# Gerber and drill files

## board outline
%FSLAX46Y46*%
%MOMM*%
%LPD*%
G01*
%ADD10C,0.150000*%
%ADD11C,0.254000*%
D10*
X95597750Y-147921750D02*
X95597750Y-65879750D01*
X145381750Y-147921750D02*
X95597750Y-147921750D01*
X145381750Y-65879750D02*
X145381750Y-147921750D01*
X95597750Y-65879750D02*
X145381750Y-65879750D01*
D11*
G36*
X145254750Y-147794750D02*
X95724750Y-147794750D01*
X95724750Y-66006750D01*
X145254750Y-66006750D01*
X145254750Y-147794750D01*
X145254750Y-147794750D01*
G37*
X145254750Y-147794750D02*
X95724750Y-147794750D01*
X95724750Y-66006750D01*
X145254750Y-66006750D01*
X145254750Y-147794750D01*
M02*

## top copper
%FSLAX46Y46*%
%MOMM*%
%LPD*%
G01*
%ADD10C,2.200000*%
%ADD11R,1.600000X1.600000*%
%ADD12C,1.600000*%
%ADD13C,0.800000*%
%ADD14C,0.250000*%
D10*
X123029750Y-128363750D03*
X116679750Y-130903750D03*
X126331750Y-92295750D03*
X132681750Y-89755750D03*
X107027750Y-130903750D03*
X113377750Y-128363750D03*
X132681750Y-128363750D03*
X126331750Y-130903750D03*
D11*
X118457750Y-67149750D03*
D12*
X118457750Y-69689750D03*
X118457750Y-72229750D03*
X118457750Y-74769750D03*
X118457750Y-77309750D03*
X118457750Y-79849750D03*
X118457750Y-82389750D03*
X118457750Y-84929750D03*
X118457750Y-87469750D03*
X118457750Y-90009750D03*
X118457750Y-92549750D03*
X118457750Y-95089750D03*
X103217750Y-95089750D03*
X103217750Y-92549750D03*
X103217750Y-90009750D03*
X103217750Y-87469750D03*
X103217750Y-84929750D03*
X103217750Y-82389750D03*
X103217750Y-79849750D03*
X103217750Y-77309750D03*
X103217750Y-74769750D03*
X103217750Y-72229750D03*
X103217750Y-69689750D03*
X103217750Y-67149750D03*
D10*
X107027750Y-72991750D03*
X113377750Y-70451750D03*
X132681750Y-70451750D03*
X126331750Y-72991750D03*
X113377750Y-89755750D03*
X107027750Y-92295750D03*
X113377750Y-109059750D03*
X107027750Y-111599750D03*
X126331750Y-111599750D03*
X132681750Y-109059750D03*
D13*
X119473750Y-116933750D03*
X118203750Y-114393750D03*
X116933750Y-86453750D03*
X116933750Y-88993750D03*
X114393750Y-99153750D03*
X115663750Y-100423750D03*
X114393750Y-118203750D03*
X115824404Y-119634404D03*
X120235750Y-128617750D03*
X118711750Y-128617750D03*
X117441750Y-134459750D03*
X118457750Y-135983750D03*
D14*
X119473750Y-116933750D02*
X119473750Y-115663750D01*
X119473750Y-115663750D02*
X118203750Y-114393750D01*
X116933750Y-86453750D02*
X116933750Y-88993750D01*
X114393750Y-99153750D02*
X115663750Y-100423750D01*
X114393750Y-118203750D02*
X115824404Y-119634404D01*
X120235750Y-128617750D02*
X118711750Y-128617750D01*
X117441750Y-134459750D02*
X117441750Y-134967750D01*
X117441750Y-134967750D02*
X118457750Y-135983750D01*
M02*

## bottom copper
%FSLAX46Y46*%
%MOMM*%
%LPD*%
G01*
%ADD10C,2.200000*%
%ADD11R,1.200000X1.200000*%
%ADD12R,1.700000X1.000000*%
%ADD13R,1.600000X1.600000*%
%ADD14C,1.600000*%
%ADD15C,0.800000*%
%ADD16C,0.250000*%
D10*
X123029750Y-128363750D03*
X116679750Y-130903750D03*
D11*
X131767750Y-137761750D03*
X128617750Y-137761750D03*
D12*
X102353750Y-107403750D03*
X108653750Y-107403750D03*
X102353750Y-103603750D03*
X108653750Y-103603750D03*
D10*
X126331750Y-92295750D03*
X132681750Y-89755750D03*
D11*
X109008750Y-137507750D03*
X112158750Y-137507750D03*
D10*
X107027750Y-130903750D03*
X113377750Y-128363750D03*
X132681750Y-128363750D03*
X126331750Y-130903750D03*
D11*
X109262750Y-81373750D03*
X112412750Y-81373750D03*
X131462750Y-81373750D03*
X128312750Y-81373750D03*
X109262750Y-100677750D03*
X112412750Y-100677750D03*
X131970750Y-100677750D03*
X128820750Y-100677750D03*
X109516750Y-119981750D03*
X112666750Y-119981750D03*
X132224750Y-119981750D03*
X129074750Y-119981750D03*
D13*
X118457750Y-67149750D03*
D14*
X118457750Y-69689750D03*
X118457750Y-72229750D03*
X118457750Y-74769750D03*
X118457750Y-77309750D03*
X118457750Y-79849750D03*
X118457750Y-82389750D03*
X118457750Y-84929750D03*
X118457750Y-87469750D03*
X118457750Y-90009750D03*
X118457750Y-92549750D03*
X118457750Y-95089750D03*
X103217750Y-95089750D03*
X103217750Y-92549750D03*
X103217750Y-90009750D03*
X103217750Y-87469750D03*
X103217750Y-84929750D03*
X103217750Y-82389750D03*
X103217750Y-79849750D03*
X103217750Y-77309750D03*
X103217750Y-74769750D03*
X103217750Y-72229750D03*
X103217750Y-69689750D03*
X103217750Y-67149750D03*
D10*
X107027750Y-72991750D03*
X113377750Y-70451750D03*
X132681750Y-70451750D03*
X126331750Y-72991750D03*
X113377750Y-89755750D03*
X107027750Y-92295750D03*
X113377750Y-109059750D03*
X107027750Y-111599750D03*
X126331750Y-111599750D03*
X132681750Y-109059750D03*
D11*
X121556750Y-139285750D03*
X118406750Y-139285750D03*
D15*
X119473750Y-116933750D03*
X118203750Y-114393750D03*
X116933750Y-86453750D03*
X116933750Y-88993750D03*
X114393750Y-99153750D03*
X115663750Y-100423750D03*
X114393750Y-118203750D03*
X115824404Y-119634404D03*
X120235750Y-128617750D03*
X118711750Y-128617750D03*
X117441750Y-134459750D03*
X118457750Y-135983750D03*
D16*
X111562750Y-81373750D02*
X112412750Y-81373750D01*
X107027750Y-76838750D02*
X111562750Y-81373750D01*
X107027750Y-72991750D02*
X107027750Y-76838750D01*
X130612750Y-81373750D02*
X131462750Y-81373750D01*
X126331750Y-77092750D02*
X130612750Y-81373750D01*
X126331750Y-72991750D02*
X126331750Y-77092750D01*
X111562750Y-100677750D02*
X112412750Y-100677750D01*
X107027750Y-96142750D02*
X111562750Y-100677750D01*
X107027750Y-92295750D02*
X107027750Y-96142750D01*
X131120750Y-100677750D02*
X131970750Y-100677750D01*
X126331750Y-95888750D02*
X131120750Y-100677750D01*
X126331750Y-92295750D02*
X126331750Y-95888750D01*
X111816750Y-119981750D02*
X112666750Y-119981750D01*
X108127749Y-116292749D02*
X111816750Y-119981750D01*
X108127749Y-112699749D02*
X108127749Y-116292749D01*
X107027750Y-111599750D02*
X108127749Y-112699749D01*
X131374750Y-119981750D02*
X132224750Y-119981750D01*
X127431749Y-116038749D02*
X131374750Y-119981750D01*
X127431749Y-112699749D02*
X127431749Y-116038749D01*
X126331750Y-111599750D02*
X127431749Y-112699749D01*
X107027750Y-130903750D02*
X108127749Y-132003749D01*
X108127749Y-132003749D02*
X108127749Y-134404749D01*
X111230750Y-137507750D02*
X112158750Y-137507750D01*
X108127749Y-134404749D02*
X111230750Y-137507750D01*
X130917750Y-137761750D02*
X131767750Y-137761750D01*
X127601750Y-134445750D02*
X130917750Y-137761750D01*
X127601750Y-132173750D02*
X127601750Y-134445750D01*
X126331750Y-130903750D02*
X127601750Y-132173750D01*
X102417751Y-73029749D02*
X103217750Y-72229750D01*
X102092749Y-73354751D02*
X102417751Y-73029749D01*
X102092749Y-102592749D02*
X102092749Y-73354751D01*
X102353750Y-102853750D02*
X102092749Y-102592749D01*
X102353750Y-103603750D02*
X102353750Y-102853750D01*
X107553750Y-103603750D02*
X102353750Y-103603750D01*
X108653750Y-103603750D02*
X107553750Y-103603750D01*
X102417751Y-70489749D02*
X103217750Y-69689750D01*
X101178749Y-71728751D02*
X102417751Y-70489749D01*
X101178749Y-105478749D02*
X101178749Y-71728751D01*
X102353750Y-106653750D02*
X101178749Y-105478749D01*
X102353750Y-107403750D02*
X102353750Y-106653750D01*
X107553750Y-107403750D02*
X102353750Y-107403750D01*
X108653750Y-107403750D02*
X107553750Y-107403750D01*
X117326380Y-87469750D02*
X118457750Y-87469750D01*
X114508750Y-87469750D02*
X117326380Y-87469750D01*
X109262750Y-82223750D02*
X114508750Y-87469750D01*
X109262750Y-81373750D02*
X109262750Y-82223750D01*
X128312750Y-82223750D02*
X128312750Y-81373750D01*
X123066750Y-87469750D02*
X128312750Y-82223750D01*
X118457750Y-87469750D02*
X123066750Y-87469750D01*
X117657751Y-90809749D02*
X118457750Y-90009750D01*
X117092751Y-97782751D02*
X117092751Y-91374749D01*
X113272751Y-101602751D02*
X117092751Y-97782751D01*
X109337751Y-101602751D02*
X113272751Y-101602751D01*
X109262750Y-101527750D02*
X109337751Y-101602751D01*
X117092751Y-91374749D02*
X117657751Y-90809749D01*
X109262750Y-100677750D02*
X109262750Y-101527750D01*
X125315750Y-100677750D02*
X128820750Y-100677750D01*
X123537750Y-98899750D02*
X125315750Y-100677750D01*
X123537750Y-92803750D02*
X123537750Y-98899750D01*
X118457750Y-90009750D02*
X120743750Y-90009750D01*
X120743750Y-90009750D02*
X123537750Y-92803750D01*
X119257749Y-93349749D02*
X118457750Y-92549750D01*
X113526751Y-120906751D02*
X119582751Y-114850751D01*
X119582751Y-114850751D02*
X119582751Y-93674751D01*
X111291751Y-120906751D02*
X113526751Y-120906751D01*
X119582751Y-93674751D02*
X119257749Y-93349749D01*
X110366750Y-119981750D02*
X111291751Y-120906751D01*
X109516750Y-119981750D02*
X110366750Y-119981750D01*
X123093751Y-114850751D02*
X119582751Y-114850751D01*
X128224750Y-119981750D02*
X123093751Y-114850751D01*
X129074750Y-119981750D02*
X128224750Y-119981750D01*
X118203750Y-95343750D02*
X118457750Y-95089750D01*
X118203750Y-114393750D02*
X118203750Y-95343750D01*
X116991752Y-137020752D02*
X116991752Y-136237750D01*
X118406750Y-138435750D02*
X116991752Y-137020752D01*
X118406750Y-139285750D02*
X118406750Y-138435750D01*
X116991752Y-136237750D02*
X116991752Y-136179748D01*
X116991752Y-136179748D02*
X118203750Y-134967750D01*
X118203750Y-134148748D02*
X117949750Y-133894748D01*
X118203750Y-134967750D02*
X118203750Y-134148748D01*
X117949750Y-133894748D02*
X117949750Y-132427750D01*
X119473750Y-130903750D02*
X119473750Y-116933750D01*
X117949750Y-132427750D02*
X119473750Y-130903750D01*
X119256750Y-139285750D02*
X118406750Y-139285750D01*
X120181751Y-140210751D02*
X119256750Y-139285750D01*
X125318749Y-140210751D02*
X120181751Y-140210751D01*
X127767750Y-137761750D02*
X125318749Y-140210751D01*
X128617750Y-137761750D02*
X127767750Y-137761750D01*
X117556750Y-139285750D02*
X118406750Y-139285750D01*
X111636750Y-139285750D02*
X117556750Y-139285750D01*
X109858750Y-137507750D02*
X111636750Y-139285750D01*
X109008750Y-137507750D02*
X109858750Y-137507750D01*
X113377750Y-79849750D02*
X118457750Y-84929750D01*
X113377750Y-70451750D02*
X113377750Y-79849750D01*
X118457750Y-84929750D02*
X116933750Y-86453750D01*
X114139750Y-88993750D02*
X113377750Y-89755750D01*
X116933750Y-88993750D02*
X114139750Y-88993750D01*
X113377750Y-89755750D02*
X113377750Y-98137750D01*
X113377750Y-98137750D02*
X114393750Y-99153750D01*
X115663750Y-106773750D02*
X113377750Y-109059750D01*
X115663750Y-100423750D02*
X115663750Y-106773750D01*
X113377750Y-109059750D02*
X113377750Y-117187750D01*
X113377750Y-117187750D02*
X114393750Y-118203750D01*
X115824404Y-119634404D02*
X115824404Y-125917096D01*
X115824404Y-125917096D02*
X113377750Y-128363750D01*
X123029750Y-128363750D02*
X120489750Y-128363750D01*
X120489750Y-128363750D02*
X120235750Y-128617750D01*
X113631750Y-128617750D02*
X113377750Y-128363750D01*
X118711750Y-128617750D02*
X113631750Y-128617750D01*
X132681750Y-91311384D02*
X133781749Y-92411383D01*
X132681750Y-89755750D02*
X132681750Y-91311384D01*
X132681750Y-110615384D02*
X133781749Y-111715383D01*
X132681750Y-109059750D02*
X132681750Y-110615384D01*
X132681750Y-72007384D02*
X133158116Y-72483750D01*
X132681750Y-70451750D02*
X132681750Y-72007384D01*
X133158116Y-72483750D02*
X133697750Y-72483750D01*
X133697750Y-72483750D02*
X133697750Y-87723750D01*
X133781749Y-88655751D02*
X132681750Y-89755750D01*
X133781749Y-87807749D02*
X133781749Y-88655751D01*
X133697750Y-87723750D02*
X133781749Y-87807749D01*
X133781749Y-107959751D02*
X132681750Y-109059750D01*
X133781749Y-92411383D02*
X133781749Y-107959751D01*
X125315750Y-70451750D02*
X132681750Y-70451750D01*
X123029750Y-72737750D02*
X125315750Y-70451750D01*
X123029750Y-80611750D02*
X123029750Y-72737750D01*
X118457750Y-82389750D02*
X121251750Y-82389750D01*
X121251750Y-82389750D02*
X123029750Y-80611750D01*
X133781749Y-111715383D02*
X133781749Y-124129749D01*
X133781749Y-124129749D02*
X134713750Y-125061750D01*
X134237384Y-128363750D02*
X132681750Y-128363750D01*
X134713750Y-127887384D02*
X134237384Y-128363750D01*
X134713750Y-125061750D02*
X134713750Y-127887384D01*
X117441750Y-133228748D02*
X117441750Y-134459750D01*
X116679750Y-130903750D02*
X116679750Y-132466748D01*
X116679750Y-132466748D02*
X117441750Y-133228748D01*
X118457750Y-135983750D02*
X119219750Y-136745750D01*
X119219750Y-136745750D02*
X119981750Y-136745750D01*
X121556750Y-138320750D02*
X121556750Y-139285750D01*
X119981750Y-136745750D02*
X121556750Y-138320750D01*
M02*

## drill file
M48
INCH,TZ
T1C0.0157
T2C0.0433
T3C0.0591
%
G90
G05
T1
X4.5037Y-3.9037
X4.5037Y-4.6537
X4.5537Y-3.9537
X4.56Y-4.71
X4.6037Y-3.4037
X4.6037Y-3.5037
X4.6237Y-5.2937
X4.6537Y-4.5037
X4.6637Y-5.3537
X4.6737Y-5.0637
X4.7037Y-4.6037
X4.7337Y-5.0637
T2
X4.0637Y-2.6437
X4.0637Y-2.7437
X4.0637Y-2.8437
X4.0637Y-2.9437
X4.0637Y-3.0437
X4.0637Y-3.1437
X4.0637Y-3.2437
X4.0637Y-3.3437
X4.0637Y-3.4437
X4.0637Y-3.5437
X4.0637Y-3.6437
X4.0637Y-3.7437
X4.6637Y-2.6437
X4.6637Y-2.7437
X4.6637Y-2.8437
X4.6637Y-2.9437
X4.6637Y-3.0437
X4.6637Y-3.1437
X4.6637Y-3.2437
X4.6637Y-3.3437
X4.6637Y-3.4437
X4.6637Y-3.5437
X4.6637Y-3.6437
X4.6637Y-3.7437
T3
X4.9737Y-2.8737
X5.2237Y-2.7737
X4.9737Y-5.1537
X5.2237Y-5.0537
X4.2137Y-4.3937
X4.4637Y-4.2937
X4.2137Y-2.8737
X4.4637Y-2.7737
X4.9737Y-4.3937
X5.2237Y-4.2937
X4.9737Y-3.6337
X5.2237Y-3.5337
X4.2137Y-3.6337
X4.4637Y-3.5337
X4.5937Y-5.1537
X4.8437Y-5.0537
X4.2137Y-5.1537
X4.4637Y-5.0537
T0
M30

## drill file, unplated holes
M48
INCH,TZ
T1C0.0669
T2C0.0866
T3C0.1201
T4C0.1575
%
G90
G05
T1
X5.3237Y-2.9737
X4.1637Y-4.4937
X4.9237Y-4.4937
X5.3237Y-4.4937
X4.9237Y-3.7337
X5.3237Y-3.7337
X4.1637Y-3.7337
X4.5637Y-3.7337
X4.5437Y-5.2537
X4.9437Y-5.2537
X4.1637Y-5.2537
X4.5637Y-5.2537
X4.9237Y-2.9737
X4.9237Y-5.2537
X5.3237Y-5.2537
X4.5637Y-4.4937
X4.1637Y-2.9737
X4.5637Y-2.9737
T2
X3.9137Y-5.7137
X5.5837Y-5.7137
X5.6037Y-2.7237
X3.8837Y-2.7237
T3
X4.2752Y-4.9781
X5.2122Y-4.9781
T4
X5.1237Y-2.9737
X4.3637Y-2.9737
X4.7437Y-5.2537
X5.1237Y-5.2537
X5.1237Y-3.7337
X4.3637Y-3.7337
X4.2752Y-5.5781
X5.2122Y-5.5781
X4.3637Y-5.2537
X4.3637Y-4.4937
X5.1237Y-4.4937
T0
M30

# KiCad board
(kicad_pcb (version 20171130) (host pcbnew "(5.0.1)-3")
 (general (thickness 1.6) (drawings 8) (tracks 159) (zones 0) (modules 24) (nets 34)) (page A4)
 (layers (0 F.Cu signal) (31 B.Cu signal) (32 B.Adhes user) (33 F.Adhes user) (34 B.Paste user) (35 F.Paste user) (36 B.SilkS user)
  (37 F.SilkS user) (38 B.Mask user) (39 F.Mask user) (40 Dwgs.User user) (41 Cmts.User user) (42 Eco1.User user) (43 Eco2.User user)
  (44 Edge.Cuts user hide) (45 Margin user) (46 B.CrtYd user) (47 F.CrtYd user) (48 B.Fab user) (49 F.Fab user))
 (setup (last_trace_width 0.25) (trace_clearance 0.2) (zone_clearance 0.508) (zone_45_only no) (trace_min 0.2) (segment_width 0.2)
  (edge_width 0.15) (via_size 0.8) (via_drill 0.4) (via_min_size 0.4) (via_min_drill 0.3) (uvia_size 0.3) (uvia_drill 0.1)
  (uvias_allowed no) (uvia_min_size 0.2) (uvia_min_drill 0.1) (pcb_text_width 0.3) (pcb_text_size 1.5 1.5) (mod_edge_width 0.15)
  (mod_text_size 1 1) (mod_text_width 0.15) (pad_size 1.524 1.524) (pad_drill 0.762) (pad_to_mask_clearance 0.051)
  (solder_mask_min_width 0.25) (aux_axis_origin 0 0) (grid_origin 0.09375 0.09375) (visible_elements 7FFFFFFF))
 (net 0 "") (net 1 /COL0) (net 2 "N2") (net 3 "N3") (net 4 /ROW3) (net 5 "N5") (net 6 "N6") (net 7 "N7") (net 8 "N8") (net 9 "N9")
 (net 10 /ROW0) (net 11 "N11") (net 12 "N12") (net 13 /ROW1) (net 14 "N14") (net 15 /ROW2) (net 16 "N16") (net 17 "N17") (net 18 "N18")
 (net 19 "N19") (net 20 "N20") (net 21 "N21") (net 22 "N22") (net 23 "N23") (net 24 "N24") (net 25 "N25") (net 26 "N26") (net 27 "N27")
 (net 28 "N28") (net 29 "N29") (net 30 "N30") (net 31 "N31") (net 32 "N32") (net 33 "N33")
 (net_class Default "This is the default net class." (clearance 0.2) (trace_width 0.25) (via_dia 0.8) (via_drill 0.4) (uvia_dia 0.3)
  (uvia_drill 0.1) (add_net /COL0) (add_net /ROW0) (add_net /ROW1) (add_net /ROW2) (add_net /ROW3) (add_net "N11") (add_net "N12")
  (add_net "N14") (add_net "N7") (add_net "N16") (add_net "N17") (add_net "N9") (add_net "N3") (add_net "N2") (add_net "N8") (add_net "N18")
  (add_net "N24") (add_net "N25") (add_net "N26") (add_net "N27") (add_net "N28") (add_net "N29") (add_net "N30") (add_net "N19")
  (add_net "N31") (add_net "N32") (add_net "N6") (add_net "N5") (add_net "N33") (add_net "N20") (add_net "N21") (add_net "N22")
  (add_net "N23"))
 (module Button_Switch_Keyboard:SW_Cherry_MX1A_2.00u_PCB (layer F.Cu) (at 123.02975 128.36375)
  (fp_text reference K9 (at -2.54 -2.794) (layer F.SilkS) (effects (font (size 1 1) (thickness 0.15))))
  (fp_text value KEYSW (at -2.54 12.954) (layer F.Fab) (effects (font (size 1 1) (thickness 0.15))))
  (pad 1 thru_hole circle (at 0 0) (size 2.2 2.2) (drill 1.5) (layers *.Cu *.Mask) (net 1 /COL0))
  (pad 2 thru_hole circle (at -6.35 2.54) (size 2.2 2.2) (drill 1.5) (layers *.Cu *.Mask) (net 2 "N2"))
  (pad "" np_thru_hole circle (at -2.54 5.08) (size 4 4) (drill 4) (layers *.Cu *.Mask))
  (pad "" np_thru_hole circle (at -7.62 5.08) (size 1.7 1.7) (drill 1.7) (layers *.Cu *.Mask))
  (pad "" np_thru_hole circle (at 2.54 5.08) (size 1.7 1.7) (drill 1.7) (layers *.Cu *.Mask))
  (pad "" np_thru_hole circle (at 9.36 13.32) (size 4 4) (drill 4) (layers *.Cu *.Mask))
  (pad "" np_thru_hole circle (at -14.44 13.32) (size 4 4) (drill 4) (layers *.Cu *.Mask))
  (pad "" np_thru_hole circle (at -14.44 -1.92) (size 3.05 3.05) (drill 3.05) (layers *.Cu *.Mask))
  (pad "" np_thru_hole circle (at 9.36 -1.92) (size 3.05 3.05) (drill 3.05) (layers *.Cu *.Mask)))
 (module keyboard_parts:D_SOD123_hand (layer B.Cu) (at 130.19275 137.76175)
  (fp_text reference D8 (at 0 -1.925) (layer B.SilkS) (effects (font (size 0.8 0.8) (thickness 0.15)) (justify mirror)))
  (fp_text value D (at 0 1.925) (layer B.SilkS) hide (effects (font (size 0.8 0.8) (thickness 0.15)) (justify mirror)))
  (pad 2 smd rect (at 1.575 0) (size 1.2 1.2) (layers B.Cu B.Paste B.Mask) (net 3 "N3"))
  (pad 1 smd rect (at -1.575 0) (size 1.2 1.2) (layers B.Cu B.Paste B.Mask) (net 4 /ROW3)))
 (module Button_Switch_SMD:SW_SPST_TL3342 (layer B.Cu) (at 105.50375 105.50375)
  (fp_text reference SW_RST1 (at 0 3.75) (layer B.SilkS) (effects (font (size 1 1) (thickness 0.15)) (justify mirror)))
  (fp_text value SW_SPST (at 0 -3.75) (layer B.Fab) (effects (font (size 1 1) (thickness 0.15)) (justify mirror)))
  (pad 1 smd rect (at -3.15 1.9) (size 1.7 1) (layers B.Cu B.Paste B.Mask) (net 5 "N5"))
  (pad 1 smd rect (at 3.15 1.9) (size 1.7 1) (layers B.Cu B.Paste B.Mask) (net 5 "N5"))
  (pad 2 smd rect (at -3.15 -1.9) (size 1.7 1) (layers B.Cu B.Paste B.Mask) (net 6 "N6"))
  (pad 2 smd rect (at 3.15 -1.9) (size 1.7 1) (layers B.Cu B.Paste B.Mask) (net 6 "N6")))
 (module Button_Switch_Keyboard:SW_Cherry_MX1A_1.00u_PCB (layer F.Cu) (at 132.68175 89.75575)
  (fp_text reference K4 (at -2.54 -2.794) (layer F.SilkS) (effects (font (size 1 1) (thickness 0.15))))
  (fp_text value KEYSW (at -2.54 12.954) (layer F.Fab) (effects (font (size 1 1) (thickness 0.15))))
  (pad "" np_thru_hole circle (at 2.54 5.08) (size 1.7 1.7) (drill 1.7) (layers *.Cu *.Mask))
  (pad "" np_thru_hole circle (at -7.62 5.08) (size 1.7 1.7) (drill 1.7) (layers *.Cu *.Mask))
  (pad "" np_thru_hole circle (at -2.54 5.08) (size 4 4) (drill 4) (layers *.Cu *.Mask))
  (pad 2 thru_hole circle (at -6.35 2.54) (size 2.2 2.2) (drill 1.5) (layers *.Cu *.Mask) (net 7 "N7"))
  (pad 1 thru_hole circle (at 0 0) (size 2.2 2.2) (drill 1.5) (layers *.Cu *.Mask) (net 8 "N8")))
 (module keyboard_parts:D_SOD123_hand (layer B.Cu) (at 110.58375 137.50775)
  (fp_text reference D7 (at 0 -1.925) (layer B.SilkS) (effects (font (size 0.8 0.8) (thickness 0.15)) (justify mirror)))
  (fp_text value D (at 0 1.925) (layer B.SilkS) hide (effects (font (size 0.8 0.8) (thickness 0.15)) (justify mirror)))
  (pad 1 smd rect (at -1.575 0) (size 1.2 1.2) (layers B.Cu B.Paste B.Mask) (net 4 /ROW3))
  (pad 2 smd rect (at 1.575 0) (size 1.2 1.2) (layers B.Cu B.Paste B.Mask) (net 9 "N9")))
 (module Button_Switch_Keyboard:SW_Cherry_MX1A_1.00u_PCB (layer F.Cu) (at 113.37775 128.36375)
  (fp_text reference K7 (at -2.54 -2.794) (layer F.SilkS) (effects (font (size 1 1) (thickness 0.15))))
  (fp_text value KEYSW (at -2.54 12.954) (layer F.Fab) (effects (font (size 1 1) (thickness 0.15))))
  (pad "" np_thru_hole circle (at 2.54 5.08) (size 1.7 1.7) (drill 1.7) (layers *.Cu *.Mask))
  (pad "" np_thru_hole circle (at -7.62 5.08) (size 1.7 1.7) (drill 1.7) (layers *.Cu *.Mask))
  (pad "" np_thru_hole circle (at -2.54 5.08) (size 4 4) (drill 4) (layers *.Cu *.Mask))
  (pad 2 thru_hole circle (at -6.35 2.54) (size 2.2 2.2) (drill 1.5) (layers *.Cu *.Mask) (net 9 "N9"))
  (pad 1 thru_hole circle (at 0 0) (size 2.2 2.2) (drill 1.5) (layers *.Cu *.Mask) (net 1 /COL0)))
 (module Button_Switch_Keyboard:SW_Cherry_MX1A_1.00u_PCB (layer F.Cu) (at 132.68175 128.36375)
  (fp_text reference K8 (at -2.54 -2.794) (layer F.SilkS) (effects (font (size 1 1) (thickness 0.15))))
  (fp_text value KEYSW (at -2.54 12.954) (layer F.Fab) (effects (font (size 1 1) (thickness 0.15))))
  (pad 1 thru_hole circle (at 0 0) (size 2.2 2.2) (drill 1.5) (layers *.Cu *.Mask) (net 8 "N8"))
  (pad 2 thru_hole circle (at -6.35 2.54) (size 2.2 2.2) (drill 1.5) (layers *.Cu *.Mask) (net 3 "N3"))
  (pad "" np_thru_hole circle (at -2.54 5.08) (size 4 4) (drill 4) (layers *.Cu *.Mask))
  (pad "" np_thru_hole circle (at -7.62 5.08) (size 1.7 1.7) (drill 1.7) (layers *.Cu *.Mask))
  (pad "" np_thru_hole circle (at 2.54 5.08) (size 1.7 1.7) (drill 1.7) (layers *.Cu *.Mask)))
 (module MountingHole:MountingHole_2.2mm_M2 (layer F.Cu) (at 99.40775 145.12775)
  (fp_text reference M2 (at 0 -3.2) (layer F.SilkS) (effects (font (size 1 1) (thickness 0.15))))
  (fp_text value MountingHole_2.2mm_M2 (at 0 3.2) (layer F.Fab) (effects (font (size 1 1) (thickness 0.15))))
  (pad 1 np_thru_hole circle (at 0 0) (size 2.2 2.2) (drill 2.2) (layers *.Cu *.Mask)))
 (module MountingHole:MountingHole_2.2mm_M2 (layer F.Cu) (at 141.82575 145.12775)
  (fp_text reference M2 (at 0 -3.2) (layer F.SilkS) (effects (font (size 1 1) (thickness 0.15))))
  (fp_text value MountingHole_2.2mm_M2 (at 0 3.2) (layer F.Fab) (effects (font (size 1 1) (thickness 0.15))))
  (pad 1 np_thru_hole circle (at 0 0) (size 2.2 2.2) (drill 2.2) (layers *.Cu *.Mask)))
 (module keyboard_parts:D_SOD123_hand (layer B.Cu) (at 110.83775 81.37375)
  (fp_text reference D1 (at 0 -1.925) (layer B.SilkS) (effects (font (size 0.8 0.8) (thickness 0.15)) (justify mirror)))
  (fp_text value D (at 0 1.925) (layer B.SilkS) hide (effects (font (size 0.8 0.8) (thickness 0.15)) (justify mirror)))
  (pad 1 smd rect (at -1.575 0) (size 1.2 1.2) (layers B.Cu B.Paste B.Mask) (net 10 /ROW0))
  (pad 2 smd rect (at 1.575 0) (size 1.2 1.2) (layers B.Cu B.Paste B.Mask) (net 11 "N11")))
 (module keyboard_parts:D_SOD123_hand (layer B.Cu) (at 129.88775 81.37375)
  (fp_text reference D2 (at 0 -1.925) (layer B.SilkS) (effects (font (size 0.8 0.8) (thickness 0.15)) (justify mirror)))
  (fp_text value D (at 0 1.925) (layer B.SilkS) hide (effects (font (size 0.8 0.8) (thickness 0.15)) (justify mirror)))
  (pad 2 smd rect (at 1.575 0) (size 1.2 1.2) (layers B.Cu B.Paste B.Mask) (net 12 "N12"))
  (pad 1 smd rect (at -1.575 0) (size 1.2 1.2) (layers B.Cu B.Paste B.Mask) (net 10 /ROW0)))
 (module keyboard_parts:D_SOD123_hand (layer B.Cu) (at 110.83775 100.67775)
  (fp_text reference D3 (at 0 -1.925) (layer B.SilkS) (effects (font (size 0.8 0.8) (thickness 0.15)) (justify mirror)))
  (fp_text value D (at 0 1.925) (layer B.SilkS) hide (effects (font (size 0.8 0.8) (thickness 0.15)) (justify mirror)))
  (pad 1 smd rect (at -1.575 0) (size 1.2 1.2) (layers B.Cu B.Paste B.Mask) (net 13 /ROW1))
  (pad 2 smd rect (at 1.575 0) (size 1.2 1.2) (layers B.Cu B.Paste B.Mask) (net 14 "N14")))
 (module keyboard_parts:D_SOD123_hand (layer B.Cu) (at 130.39575 100.67775)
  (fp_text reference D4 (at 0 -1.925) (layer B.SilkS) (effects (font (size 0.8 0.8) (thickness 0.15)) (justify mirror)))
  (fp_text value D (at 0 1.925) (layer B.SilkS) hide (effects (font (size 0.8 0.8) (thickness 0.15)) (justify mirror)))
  (pad 2 smd rect (at 1.575 0) (size 1.2 1.2) (layers B.Cu B.Paste B.Mask) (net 7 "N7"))
  (pad 1 smd rect (at -1.575 0) (size 1.2 1.2) (layers B.Cu B.Paste B.Mask) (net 13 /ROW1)))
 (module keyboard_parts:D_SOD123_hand (layer B.Cu) (at 111.09175 119.98175)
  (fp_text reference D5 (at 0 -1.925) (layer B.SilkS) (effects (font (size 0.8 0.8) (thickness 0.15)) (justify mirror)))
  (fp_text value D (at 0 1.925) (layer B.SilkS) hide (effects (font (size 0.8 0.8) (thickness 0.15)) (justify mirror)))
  (pad 1 smd rect (at -1.575 0) (size 1.2 1.2) (layers B.Cu B.Paste B.Mask) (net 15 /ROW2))
  (pad 2 smd rect (at 1.575 0) (size 1.2 1.2) (layers B.Cu B.Paste B.Mask) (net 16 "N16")))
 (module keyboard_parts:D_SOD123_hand (layer B.Cu) (at 130.64975 119.98175)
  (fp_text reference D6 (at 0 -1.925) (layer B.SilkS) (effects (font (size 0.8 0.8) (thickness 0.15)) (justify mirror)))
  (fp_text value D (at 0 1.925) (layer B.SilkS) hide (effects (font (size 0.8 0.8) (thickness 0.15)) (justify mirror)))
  (pad 2 smd rect (at 1.575 0) (size 1.2 1.2) (layers B.Cu B.Paste B.Mask) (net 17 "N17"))
  (pad 1 smd rect (at -1.575 0) (size 1.2 1.2) (layers B.Cu B.Paste B.Mask) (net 15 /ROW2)))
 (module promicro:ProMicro (layer B.Cu) (at 110.83775 81.11975 270)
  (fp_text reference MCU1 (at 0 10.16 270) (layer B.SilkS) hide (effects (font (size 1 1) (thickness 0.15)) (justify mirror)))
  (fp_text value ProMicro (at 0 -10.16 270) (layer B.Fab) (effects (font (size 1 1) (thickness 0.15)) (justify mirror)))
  (pad 1 thru_hole rect (at -13.97 -7.62 270) (size 1.6 1.6) (drill 1.1) (layers *.Cu *.Mask B.SilkS) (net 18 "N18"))
  (pad 2 thru_hole circle (at -11.43 -7.62 270) (size 1.6 1.6) (drill 1.1) (layers *.Cu *.Mask B.SilkS) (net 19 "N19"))
  (pad 3 thru_hole circle (at -8.89 -7.62 270) (size 1.6 1.6) (drill 1.1) (layers *.Cu *.Mask B.SilkS) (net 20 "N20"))
  (pad 4 thru_hole circle (at -6.35 -7.62 270) (size 1.6 1.6) (drill 1.1) (layers *.Cu *.Mask B.SilkS) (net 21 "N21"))
  (pad 5 thru_hole circle (at -3.81 -7.62 270) (size 1.6 1.6) (drill 1.1) (layers *.Cu *.Mask B.SilkS) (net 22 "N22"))
  (pad 6 thru_hole circle (at -1.27 -7.62 270) (size 1.6 1.6) (drill 1.1) (layers *.Cu *.Mask B.SilkS) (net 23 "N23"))
  (pad 7 thru_hole circle (at 1.27 -7.62 270) (size 1.6 1.6) (drill 1.1) (layers *.Cu *.Mask B.SilkS) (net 8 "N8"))
  (pad 8 thru_hole circle (at 3.81 -7.62 270) (size 1.6 1.6) (drill 1.1) (layers *.Cu *.Mask B.SilkS) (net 1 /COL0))
  (pad 9 thru_hole circle (at 6.35 -7.62 270) (size 1.6 1.6) (drill 1.1) (layers *.Cu *.Mask B.SilkS) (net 10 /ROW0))
  (pad 10 thru_hole circle (at 8.89 -7.62 270) (size 1.6 1.6) (drill 1.1) (layers *.Cu *.Mask B.SilkS) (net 13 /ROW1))
  (pad 11 thru_hole circle (at 11.43 -7.62 270) (size 1.6 1.6) (drill 1.1) (layers *.Cu *.Mask B.SilkS) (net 15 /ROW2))
  (pad 12 thru_hole circle (at 13.97 -7.62 270) (size 1.6 1.6) (drill 1.1) (layers *.Cu *.Mask B.SilkS) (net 4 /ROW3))
  (pad 13 thru_hole circle (at 13.97 7.62 270) (size 1.6 1.6) (drill 1.1) (layers *.Cu *.Mask B.SilkS) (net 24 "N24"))
  (pad 14 thru_hole circle (at 11.43 7.62 270) (size 1.6 1.6) (drill 1.1) (layers *.Cu *.Mask B.SilkS) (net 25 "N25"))
  (pad 15 thru_hole circle (at 8.89 7.62 270) (size 1.6 1.6) (drill 1.1) (layers *.Cu *.Mask B.SilkS) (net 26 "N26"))
  (pad 16 thru_hole circle (at 6.35 7.62 270) (size 1.6 1.6) (drill 1.1) (layers *.Cu *.Mask B.SilkS) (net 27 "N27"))
  (pad 17 thru_hole circle (at 3.81 7.62 270) (size 1.6 1.6) (drill 1.1) (layers *.Cu *.Mask B.SilkS) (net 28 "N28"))
  (pad 18 thru_hole circle (at 1.27 7.62 270) (size 1.6 1.6) (drill 1.1) (layers *.Cu *.Mask B.SilkS) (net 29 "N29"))
  (pad 19 thru_hole circle (at -1.27 7.62 270) (size 1.6 1.6) (drill 1.1) (layers *.Cu *.Mask B.SilkS) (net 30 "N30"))
  (pad 20 thru_hole circle (at -3.81 7.62 270) (size 1.6 1.6) (drill 1.1) (layers *.Cu *.Mask B.SilkS) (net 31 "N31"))
  (pad 21 thru_hole circle (at -6.35 7.62 270) (size 1.6 1.6) (drill 1.1) (layers *.Cu *.Mask B.SilkS) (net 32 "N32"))
  (pad 22 thru_hole circle (at -8.89 7.62 270) (size 1.6 1.6) (drill 1.1) (layers *.Cu *.Mask B.SilkS) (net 6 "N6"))
  (pad 23 thru_hole circle (at -11.43 7.62 270) (size 1.6 1.6) (drill 1.1) (layers *.Cu *.Mask B.SilkS) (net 5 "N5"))
  (pad 24 thru_hole circle (at -13.97 7.62 270) (size 1.6 1.6) (drill 1.1) (layers *.Cu *.Mask B.SilkS) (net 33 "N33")))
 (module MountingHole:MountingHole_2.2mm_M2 (layer F.Cu) (at 142.33375 69.18175)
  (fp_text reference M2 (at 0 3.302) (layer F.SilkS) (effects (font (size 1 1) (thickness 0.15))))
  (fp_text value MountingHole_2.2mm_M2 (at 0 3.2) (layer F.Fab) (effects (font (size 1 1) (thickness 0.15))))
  (pad 1 np_thru_hole circle (at 0 0) (size 2.2 2.2) (drill 2.2) (layers *.Cu *.Mask)))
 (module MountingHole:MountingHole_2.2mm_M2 (layer F.Cu) (at 98.64575 69.18175)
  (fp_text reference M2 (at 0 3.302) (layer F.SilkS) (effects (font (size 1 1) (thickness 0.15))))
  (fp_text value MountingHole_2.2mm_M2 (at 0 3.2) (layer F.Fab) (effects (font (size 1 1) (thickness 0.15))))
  (pad 1 np_thru_hole circle (at 0 0) (size 2.2 2.2) (drill 2.2) (layers *.Cu *.Mask)))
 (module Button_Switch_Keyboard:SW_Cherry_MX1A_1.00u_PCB (layer F.Cu) (at 113.37775 70.45175)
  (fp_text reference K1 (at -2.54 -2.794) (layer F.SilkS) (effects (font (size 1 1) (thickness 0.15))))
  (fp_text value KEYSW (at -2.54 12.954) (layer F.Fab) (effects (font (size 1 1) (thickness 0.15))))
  (pad "" np_thru_hole circle (at 2.54 5.08) (size 1.7 1.7) (drill 1.7) (layers *.Cu *.Mask))
  (pad "" np_thru_hole circle (at -7.62 5.08) (size 1.7 1.7) (drill 1.7) (layers *.Cu *.Mask))
  (pad "" np_thru_hole circle (at -2.54 5.08) (size 4 4) (drill 4) (layers *.Cu *.Mask))
  (pad 2 thru_hole circle (at -6.35 2.54) (size 2.2 2.2) (drill 1.5) (layers *.Cu *.Mask) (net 11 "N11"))
  (pad 1 thru_hole circle (at 0 0) (size 2.2 2.2) (drill 1.5) (layers *.Cu *.Mask) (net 1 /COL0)))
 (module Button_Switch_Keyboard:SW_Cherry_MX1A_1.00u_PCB (layer F.Cu) (at 132.68175 70.45175)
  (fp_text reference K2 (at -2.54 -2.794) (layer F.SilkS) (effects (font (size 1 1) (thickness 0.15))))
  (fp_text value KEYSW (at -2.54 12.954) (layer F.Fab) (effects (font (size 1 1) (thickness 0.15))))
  (pad 1 thru_hole circle (at 0 0) (size 2.2 2.2) (drill 1.5) (layers *.Cu *.Mask) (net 8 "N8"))
  (pad 2 thru_hole circle (at -6.35 2.54) (size 2.2 2.2) (drill 1.5) (layers *.Cu *.Mask) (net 12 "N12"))
  (pad "" np_thru_hole circle (at -2.54 5.08) (size 4 4) (drill 4) (layers *.Cu *.Mask))
  (pad "" np_thru_hole circle (at -7.62 5.08) (size 1.7 1.7) (drill 1.7) (layers *.Cu *.Mask))
  (pad "" np_thru_hole circle (at 2.54 5.08) (size 1.7 1.7) (drill 1.7) (layers *.Cu *.Mask)))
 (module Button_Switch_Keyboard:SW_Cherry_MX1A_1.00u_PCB (layer F.Cu) (at 113.37775 89.75575)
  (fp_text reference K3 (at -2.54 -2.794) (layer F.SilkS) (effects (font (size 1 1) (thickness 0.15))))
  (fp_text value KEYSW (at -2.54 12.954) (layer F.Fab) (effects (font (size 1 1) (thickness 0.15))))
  (pad 1 thru_hole circle (at 0 0) (size 2.2 2.2) (drill 1.5) (layers *.Cu *.Mask) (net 1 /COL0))
  (pad 2 thru_hole circle (at -6.35 2.54) (size 2.2 2.2) (drill 1.5) (layers *.Cu *.Mask) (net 14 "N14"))
  (pad "" np_thru_hole circle (at -2.54 5.08) (size 4 4) (drill 4) (layers *.Cu *.Mask))
  (pad "" np_thru_hole circle (at -7.62 5.08) (size 1.7 1.7) (drill 1.7) (layers *.Cu *.Mask))
  (pad "" np_thru_hole circle (at 2.54 5.08) (size 1.7 1.7) (drill 1.7) (layers *.Cu *.Mask)))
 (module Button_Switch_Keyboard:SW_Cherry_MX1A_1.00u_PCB (layer F.Cu) (at 113.37775 109.05975)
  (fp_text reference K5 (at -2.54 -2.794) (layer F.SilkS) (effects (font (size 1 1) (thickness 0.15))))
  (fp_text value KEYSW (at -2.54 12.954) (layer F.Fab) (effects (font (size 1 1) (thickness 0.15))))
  (pad 1 thru_hole circle (at 0 0) (size 2.2 2.2) (drill 1.5) (layers *.Cu *.Mask) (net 1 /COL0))
  (pad 2 thru_hole circle (at -6.35 2.54) (size 2.2 2.2) (drill 1.5) (layers *.Cu *.Mask) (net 16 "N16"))
  (pad "" np_thru_hole circle (at -2.54 5.08) (size 4 4) (drill 4) (layers *.Cu *.Mask))
  (pad "" np_thru_hole circle (at -7.62 5.08) (size 1.7 1.7) (drill 1.7) (layers *.Cu *.Mask))
  (pad "" np_thru_hole circle (at 2.54 5.08) (size 1.7 1.7) (drill 1.7) (layers *.Cu *.Mask)))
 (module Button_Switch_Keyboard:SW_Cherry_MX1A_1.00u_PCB (layer F.Cu) (at 132.68175 109.05975)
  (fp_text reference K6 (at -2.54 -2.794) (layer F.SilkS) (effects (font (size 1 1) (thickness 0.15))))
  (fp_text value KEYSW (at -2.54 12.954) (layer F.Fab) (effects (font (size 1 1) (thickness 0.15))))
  (pad "" np_thru_hole circle (at 2.54 5.08) (size 1.7 1.7) (drill 1.7) (layers *.Cu *.Mask))
  (pad "" np_thru_hole circle (at -7.62 5.08) (size 1.7 1.7) (drill 1.7) (layers *.Cu *.Mask))
  (pad "" np_thru_hole circle (at -2.54 5.08) (size 4 4) (drill 4) (layers *.Cu *.Mask))
  (pad 2 thru_hole circle (at -6.35 2.54) (size 2.2 2.2) (drill 1.5) (layers *.Cu *.Mask) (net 17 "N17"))
  (pad 1 thru_hole circle (at 0 0) (size 2.2 2.2) (drill 1.5) (layers *.Cu *.Mask) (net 8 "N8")))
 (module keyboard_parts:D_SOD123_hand (layer B.Cu) (at 119.98175 139.28575)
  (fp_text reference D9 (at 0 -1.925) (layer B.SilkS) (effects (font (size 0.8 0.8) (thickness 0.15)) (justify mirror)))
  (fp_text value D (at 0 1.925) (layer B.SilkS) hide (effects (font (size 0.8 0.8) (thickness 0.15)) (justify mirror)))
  (pad 2 smd rect (at 1.575 0) (size 1.2 1.2) (layers B.Cu B.Paste B.Mask) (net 2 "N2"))
  (pad 1 smd rect (at -1.575 0) (size 1.2 1.2) (layers B.Cu B.Paste B.Mask) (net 4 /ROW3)))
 (gr_line (start 95.59775 147.92175) (end 95.59775 65.87975) (layer Edge.Cuts) (width 0.15))
 (gr_line (start 145.38175 147.92175) (end 95.59775 147.92175) (layer Edge.Cuts) (width 0.15))
 (gr_line (start 145.38175 65.87975) (end 145.38175 147.92175) (layer Edge.Cuts) (width 0.15))
 (gr_line (start 95.59775 65.87975) (end 145.38175 65.87975) (layer Edge.Cuts) (width 0.15))
 (segment (start 111.56275 81.37375) (end 112.41275 81.37375) (width 0.25) (layer B.Cu) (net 11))
 (segment (start 107.02775 76.83875) (end 111.56275 81.37375) (width 0.25) (layer B.Cu) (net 11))
 (segment (start 107.02775 72.99175) (end 107.02775 76.83875) (width 0.25) (layer B.Cu) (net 11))
 (segment (start 130.61275 81.37375) (end 131.46275 81.37375) (width 0.25) (layer B.Cu) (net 12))
 (segment (start 126.33175 77.09275) (end 130.61275 81.37375) (width 0.25) (layer B.Cu) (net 12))
 (segment (start 126.33175 72.99175) (end 126.33175 77.09275) (width 0.25) (layer B.Cu) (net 12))
 (segment (start 111.56275 100.67775) (end 112.41275 100.67775) (width 0.25) (layer B.Cu) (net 14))
 (segment (start 107.02775 96.14275) (end 111.56275 100.67775) (width 0.25) (layer B.Cu) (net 14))
 (segment (start 107.02775 92.29575) (end 107.02775 96.14275) (width 0.25) (layer B.Cu) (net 14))
 (segment (start 131.12075 100.67775) (end 131.97075 100.67775) (width 0.25) (layer B.Cu) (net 7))
 (segment (start 126.33175 95.88875) (end 131.12075 100.67775) (width 0.25) (layer B.Cu) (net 7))
 (segment (start 126.33175 92.29575) (end 126.33175 95.88875) (width 0.25) (layer B.Cu) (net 7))
 (segment (start 111.81675 119.98175) (end 112.66675 119.98175) (width 0.25) (layer B.Cu) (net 16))
 (segment (start 108.127749 116.292749) (end 111.81675 119.98175) (width 0.25) (layer B.Cu) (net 16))
 (segment (start 108.127749 112.699749) (end 108.127749 116.292749) (width 0.25) (layer B.Cu) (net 16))
 (segment (start 107.02775 111.59975) (end 108.127749 112.699749) (width 0.25) (layer B.Cu) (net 16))
 (segment (start 131.37475 119.98175) (end 132.22475 119.98175) (width 0.25) (layer B.Cu) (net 17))
 (segment (start 127.431749 116.038749) (end 131.37475 119.98175) (width 0.25) (layer B.Cu) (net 17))
 (segment (start 127.431749 112.699749) (end 127.431749 116.038749) (width 0.25) (layer B.Cu) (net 17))
 (segment (start 126.33175 111.59975) (end 127.431749 112.699749) (width 0.25) (layer B.Cu) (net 17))
 (segment (start 107.02775 130.90375) (end 108.127749 132.003749) (width 0.25) (layer B.Cu) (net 9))
 (segment (start 108.127749 132.003749) (end 108.127749 134.404749) (width 0.25) (layer B.Cu) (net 9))
 (segment (start 111.23075 137.50775) (end 112.15875 137.50775) (width 0.25) (layer B.Cu) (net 9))
 (segment (start 108.127749 134.404749) (end 111.23075 137.50775) (width 0.25) (layer B.Cu) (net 9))
 (segment (start 130.91775 137.76175) (end 131.76775 137.76175) (width 0.25) (layer B.Cu) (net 3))
 (segment (start 127.60175 134.44575) (end 130.91775 137.76175) (width 0.25) (layer B.Cu) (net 3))
 (segment (start 127.60175 132.17375) (end 127.60175 134.44575) (width 0.25) (layer B.Cu) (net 3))
 (segment (start 126.33175 130.90375) (end 127.60175 132.17375) (width 0.25) (layer B.Cu) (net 3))
 (segment (start 102.417751 73.029749) (end 103.21775 72.22975) (width 0.25) (layer B.Cu) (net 6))
 (segment (start 102.092749 73.354751) (end 102.417751 73.029749) (width 0.25) (layer B.Cu) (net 6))
 (segment (start 102.092749 102.592749) (end 102.092749 73.354751) (width 0.25) (layer B.Cu) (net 6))
 (segment (start 102.35375 102.85375) (end 102.092749 102.592749) (width 0.25) (layer B.Cu) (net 6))
 (segment (start 102.35375 103.60375) (end 102.35375 102.85375) (width 0.25) (layer B.Cu) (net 6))
 (segment (start 107.55375 103.60375) (end 102.35375 103.60375) (width 0.25) (layer B.Cu) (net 6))
 (segment (start 108.65375 103.60375) (end 107.55375 103.60375) (width 0.25) (layer B.Cu) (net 6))
 (segment (start 102.417751 70.489749) (end 103.21775 69.68975) (width 0.25) (layer B.Cu) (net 5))
 (segment (start 101.178749 71.728751) (end 102.417751 70.489749) (width 0.25) (layer B.Cu) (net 5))
 (segment (start 101.178749 105.478749) (end 101.178749 71.728751) (width 0.25) (layer B.Cu) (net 5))
 (segment (start 102.35375 106.65375) (end 101.178749 105.478749) (width 0.25) (layer B.Cu) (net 5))
 (segment (start 102.35375 107.40375) (end 102.35375 106.65375) (width 0.25) (layer B.Cu) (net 5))
 (segment (start 107.55375 107.40375) (end 102.35375 107.40375) (width 0.25) (layer B.Cu) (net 5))
 (segment (start 108.65375 107.40375) (end 107.55375 107.40375) (width 0.25) (layer B.Cu) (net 5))
 (segment (start 117.32638 87.46975) (end 118.45775 87.46975) (width 0.25) (layer B.Cu) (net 10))
 (segment (start 114.50875 87.46975) (end 117.32638 87.46975) (width 0.25) (layer B.Cu) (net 10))
 (segment (start 109.26275 82.22375) (end 114.50875 87.46975) (width 0.25) (layer B.Cu) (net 10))
 (segment (start 109.26275 81.37375) (end 109.26275 82.22375) (width 0.25) (layer B.Cu) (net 10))
 (segment (start 128.31275 82.22375) (end 128.31275 81.37375) (width 0.25) (layer B.Cu) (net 10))
 (segment (start 123.06675 87.46975) (end 128.31275 82.22375) (width 0.25) (layer B.Cu) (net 10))
 (segment (start 118.45775 87.46975) (end 123.06675 87.46975) (width 0.25) (layer B.Cu) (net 10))
 (segment (start 117.657751 90.809749) (end 118.45775 90.00975) (width 0.25) (layer B.Cu) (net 13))
 (segment (start 117.092751 97.782751) (end 117.092751 91.374749) (width 0.25) (layer B.Cu) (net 13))
 (segment (start 113.272751 101.602751) (end 117.092751 97.782751) (width 0.25) (layer B.Cu) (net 13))
 (segment (start 109.337751 101.602751) (end 113.272751 101.602751) (width 0.25) (layer B.Cu) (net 13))
 (segment (start 109.26275 101.52775) (end 109.337751 101.602751) (width 0.25) (layer B.Cu) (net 13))
 (segment (start 117.092751 91.374749) (end 117.657751 90.809749) (width 0.25) (layer B.Cu) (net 13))
 (segment (start 109.26275 100.67775) (end 109.26275 101.52775) (width 0.25) (layer B.Cu) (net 13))
 (segment (start 125.31575 100.67775) (end 128.82075 100.67775) (width 0.25) (layer B.Cu) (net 13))
 (segment (start 123.53775 98.89975) (end 125.31575 100.67775) (width 0.25) (layer B.Cu) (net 13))
 (segment (start 123.53775 92.80375) (end 123.53775 98.89975) (width 0.25) (layer B.Cu) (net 13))
 (segment (start 118.45775 90.00975) (end 120.74375 90.00975) (width 0.25) (layer B.Cu) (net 13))
 (segment (start 120.74375 90.00975) (end 123.53775 92.80375) (width 0.25) (layer B.Cu) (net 13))
 (segment (start 119.257749 93.349749) (end 118.45775 92.54975) (width 0.25) (layer B.Cu) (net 15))
 (segment (start 113.526751 120.906751) (end 119.582751 114.850751) (width 0.25) (layer B.Cu) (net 15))
 (segment (start 119.582751 114.850751) (end 119.582751 93.674751) (width 0.25) (layer B.Cu) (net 15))
 (segment (start 111.291751 120.906751) (end 113.526751 120.906751) (width 0.25) (layer B.Cu) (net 15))
 (segment (start 119.582751 93.674751) (end 119.257749 93.349749) (width 0.25) (layer B.Cu) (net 15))
 (segment (start 110.36675 119.98175) (end 111.291751 120.906751) (width 0.25) (layer B.Cu) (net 15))
 (segment (start 109.51675 119.98175) (end 110.36675 119.98175) (width 0.25) (layer B.Cu) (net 15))
 (segment (start 123.093751 114.850751) (end 119.582751 114.850751) (width 0.25) (layer B.Cu) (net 15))
 (segment (start 128.22475 119.98175) (end 123.093751 114.850751) (width 0.25) (layer B.Cu) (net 15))
 (segment (start 129.07475 119.98175) (end 128.22475 119.98175) (width 0.25) (layer B.Cu) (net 15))
 (via (at 119.47375 116.93375) (size 0.8) (drill 0.4) (layers F.Cu B.Cu) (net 4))
 (segment (start 119.47375 116.93375) (end 119.47375 115.66375) (width 0.25) (layer F.Cu) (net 4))
 (segment (start 119.47375 115.66375) (end 118.20375 114.39375) (width 0.25) (layer F.Cu) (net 4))
 (via (at 118.20375 114.39375) (size 0.8) (drill 0.4) (layers F.Cu B.Cu) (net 4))
 (segment (start 118.20375 95.34375) (end 118.45775 95.08975) (width 0.25) (layer B.Cu) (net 4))
 (segment (start 118.20375 114.39375) (end 118.20375 95.34375) (width 0.25) (layer B.Cu) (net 4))
 (segment (start 116.991752 137.020752) (end 116.991752 136.23775) (width 0.25) (layer B.Cu) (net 4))
 (segment (start 118.40675 138.43575) (end 116.991752 137.020752) (width 0.25) (layer B.Cu) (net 4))
 (segment (start 118.40675 139.28575) (end 118.40675 138.43575) (width 0.25) (layer B.Cu) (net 4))
 (segment (start 116.991752 136.23775) (end 116.991752 136.179748) (width 0.25) (layer B.Cu) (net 4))
 (segment (start 116.991752 136.179748) (end 118.20375 134.96775) (width 0.25) (layer B.Cu) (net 4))
 (segment (start 118.20375 134.148748) (end 117.94975 133.894748) (width 0.25) (layer B.Cu) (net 4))
 (segment (start 118.20375 134.96775) (end 118.20375 134.148748) (width 0.25) (layer B.Cu) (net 4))
 (segment (start 117.94975 133.894748) (end 117.94975 132.42775) (width 0.25) (layer B.Cu) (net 4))
 (segment (start 119.47375 130.90375) (end 119.47375 116.93375) (width 0.25) (layer B.Cu) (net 4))
 (segment (start 117.94975 132.42775) (end 119.47375 130.90375) (width 0.25) (layer B.Cu) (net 4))
 (segment (start 119.25675 139.28575) (end 118.40675 139.28575) (width 0.25) (layer B.Cu) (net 4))
 (segment (start 120.181751 140.210751) (end 119.25675 139.28575) (width 0.25) (layer B.Cu) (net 4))
 (segment (start 125.318749 140.210751) (end 120.181751 140.210751) (width 0.25) (layer B.Cu) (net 4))
 (segment (start 127.76775 137.76175) (end 125.318749 140.210751) (width 0.25) (layer B.Cu) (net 4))
 (segment (start 128.61775 137.76175) (end 127.76775 137.76175) (width 0.25) (layer B.Cu) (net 4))
 (segment (start 117.55675 139.28575) (end 118.40675 139.28575) (width 0.25) (layer B.Cu) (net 4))
 (segment (start 111.63675 139.28575) (end 117.55675 139.28575) (width 0.25) (layer B.Cu) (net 4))
 (segment (start 109.85875 137.50775) (end 111.63675 139.28575) (width 0.25) (layer B.Cu) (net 4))
 (segment (start 109.00875 137.50775) (end 109.85875 137.50775) (width 0.25) (layer B.Cu) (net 4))
 (segment (start 113.37775 79.84975) (end 118.45775 84.92975) (width 0.25) (layer B.Cu) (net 1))
 (segment (start 113.37775 70.45175) (end 113.37775 79.84975) (width 0.25) (layer B.Cu) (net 1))
 (via (at 116.93375 86.45375) (size 0.8) (drill 0.4) (layers F.Cu B.Cu) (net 1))
 (segment (start 118.45775 84.92975) (end 116.93375 86.45375) (width 0.25) (layer B.Cu) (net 1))
 (via (at 116.93375 88.99375) (size 0.8) (drill 0.4) (layers F.Cu B.Cu) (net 1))
 (segment (start 116.93375 86.45375) (end 116.93375 88.99375) (width 0.25) (layer F.Cu) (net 1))
 (segment (start 114.13975 88.99375) (end 113.37775 89.75575) (width 0.25) (layer B.Cu) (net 1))
 (segment (start 116.93375 88.99375) (end 114.13975 88.99375) (width 0.25) (layer B.Cu) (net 1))
 (via (at 114.39375 99.15375) (size 0.8) (drill 0.4) (layers F.Cu B.Cu) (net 1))
 (segment (start 113.37775 89.75575) (end 113.37775 98.13775) (width 0.25) (layer B.Cu) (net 1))
 (segment (start 113.37775 98.13775) (end 114.39375 99.15375) (width 0.25) (layer B.Cu) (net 1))
 (segment (start 114.39375 99.15375) (end 115.66375 100.42375) (width 0.25) (layer F.Cu) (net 1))
 (via (at 115.66375 100.42375) (size 0.8) (drill 0.4) (layers F.Cu B.Cu) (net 1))
 (segment (start 115.66375 106.77375) (end 113.37775 109.05975) (width 0.25) (layer B.Cu) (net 1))
 (segment (start 115.66375 100.42375) (end 115.66375 106.77375) (width 0.25) (layer B.Cu) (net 1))
 (via (at 114.39375 118.20375) (size 0.8) (drill 0.4) (layers F.Cu B.Cu) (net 1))
 (segment (start 113.37775 109.05975) (end 113.37775 117.18775) (width 0.25) (layer B.Cu) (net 1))
 (segment (start 113.37775 117.18775) (end 114.39375 118.20375) (width 0.25) (layer B.Cu) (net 1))
 (via (at 115.824404 119.634404) (size 0.8) (drill 0.4) (layers F.Cu B.Cu) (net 1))
 (segment (start 114.39375 118.20375) (end 115.824404 119.634404) (width 0.25) (layer F.Cu) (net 1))
 (segment (start 115.824404 119.634404) (end 115.824404 125.917096) (width 0.25) (layer B.Cu) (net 1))
 (segment (start 115.824404 125.917096) (end 113.37775 128.36375) (width 0.25) (layer B.Cu) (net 1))
 (via (at 120.23575 128.61775) (size 0.8) (drill 0.4) (layers F.Cu B.Cu) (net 1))
 (segment (start 123.02975 128.36375) (end 120.48975 128.36375) (width 0.25) (layer B.Cu) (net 1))
 (segment (start 120.48975 128.36375) (end 120.23575 128.61775) (width 0.25) (layer B.Cu) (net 1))
 (via (at 118.71175 128.61775) (size 0.8) (drill 0.4) (layers F.Cu B.Cu) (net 1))
 (segment (start 120.23575 128.61775) (end 118.71175 128.61775) (width 0.25) (layer F.Cu) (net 1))
 (segment (start 113.63175 128.61775) (end 113.37775 128.36375) (width 0.25) (layer B.Cu) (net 1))
 (segment (start 118.71175 128.61775) (end 113.63175 128.61775) (width 0.25) (layer B.Cu) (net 1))
 (segment (start 132.68175 91.311384) (end 133.781749 92.411383) (width 0.25) (layer B.Cu) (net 8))
 (segment (start 132.68175 89.75575) (end 132.68175 91.311384) (width 0.25) (layer B.Cu) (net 8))
 (segment (start 132.68175 110.615384) (end 133.781749 111.715383) (width 0.25) (layer B.Cu) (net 8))
 (segment (start 132.68175 109.05975) (end 132.68175 110.615384) (width 0.25) (layer B.Cu) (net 8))
 (segment (start 132.68175 72.007384) (end 133.158116 72.48375) (width 0.25) (layer B.Cu) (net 8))
 (segment (start 132.68175 70.45175) (end 132.68175 72.007384) (width 0.25) (layer B.Cu) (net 8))
 (segment (start 133.158116 72.48375) (end 133.69775 72.48375) (width 0.25) (layer B.Cu) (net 8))
 (segment (start 133.69775 72.48375) (end 133.69775 87.72375) (width 0.25) (layer B.Cu) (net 8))
 (segment (start 133.781749 88.655751) (end 132.68175 89.75575) (width 0.25) (layer B.Cu) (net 8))
 (segment (start 133.781749 87.807749) (end 133.781749 88.655751) (width 0.25) (layer B.Cu) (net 8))
 (segment (start 133.69775 87.72375) (end 133.781749 87.807749) (width 0.25) (layer B.Cu) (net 8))
 (segment (start 133.781749 107.959751) (end 132.68175 109.05975) (width 0.25) (layer B.Cu) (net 8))
 (segment (start 133.781749 92.411383) (end 133.781749 107.959751) (width 0.25) (layer B.Cu) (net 8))
 (segment (start 125.31575 70.45175) (end 132.68175 70.45175) (width 0.25) (layer B.Cu) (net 8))
 (segment (start 123.02975 72.73775) (end 125.31575 70.45175) (width 0.25) (layer B.Cu) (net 8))
 (segment (start 123.02975 80.61175) (end 123.02975 72.73775) (width 0.25) (layer B.Cu) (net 8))
 (segment (start 118.45775 82.38975) (end 121.25175 82.38975) (width 0.25) (layer B.Cu) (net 8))
 (segment (start 121.25175 82.38975) (end 123.02975 80.61175) (width 0.25) (layer B.Cu) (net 8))
 (segment (start 133.781749 111.715383) (end 133.781749 124.129749) (width 0.25) (layer B.Cu) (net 8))
 (segment (start 133.781749 124.129749) (end 134.71375 125.06175) (width 0.25) (layer B.Cu) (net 8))
 (segment (start 134.237384 128.36375) (end 132.68175 128.36375) (width 0.25) (layer B.Cu) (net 8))
 (segment (start 134.71375 127.887384) (end 134.237384 128.36375) (width 0.25) (layer B.Cu) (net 8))
 (segment (start 134.71375 125.06175) (end 134.71375 127.887384) (width 0.25) (layer B.Cu) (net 8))
 (via (at 117.44175 134.45975) (size 0.8) (drill 0.4) (layers F.Cu B.Cu) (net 2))
 (segment (start 117.44175 133.228748) (end 117.44175 134.45975) (width 0.25) (layer B.Cu) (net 2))
 (segment (start 116.67975 130.90375) (end 116.67975 132.466748) (width 0.25) (layer B.Cu) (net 2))
 (segment (start 116.67975 132.466748) (end 117.44175 133.228748) (width 0.25) (layer B.Cu) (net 2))
 (via (at 118.45775 135.98375) (size 0.8) (drill 0.4) (layers F.Cu B.Cu) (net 2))
 (segment (start 117.44175 134.45975) (end 117.44175 134.96775) (width 0.25) (layer F.Cu) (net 2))
 (segment (start 117.44175 134.96775) (end 118.45775 135.98375) (width 0.25) (layer F.Cu) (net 2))
 (segment (start 118.45775 135.98375) (end 119.21975 136.74575) (width 0.25) (layer B.Cu) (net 2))
 (segment (start 119.21975 136.74575) (end 119.98175 136.74575) (width 0.25) (layer B.Cu) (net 2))
 (segment (start 121.55675 138.32075) (end 121.55675 139.28575) (width 0.25) (layer B.Cu) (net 2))
 (segment (start 119.98175 136.74575) (end 121.55675 138.32075) (width 0.25) (layer B.Cu) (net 2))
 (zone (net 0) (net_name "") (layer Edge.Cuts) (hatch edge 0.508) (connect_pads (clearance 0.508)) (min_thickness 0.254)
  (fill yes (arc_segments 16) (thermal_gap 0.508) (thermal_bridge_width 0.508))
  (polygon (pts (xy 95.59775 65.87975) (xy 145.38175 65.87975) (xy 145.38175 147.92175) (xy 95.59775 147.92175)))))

